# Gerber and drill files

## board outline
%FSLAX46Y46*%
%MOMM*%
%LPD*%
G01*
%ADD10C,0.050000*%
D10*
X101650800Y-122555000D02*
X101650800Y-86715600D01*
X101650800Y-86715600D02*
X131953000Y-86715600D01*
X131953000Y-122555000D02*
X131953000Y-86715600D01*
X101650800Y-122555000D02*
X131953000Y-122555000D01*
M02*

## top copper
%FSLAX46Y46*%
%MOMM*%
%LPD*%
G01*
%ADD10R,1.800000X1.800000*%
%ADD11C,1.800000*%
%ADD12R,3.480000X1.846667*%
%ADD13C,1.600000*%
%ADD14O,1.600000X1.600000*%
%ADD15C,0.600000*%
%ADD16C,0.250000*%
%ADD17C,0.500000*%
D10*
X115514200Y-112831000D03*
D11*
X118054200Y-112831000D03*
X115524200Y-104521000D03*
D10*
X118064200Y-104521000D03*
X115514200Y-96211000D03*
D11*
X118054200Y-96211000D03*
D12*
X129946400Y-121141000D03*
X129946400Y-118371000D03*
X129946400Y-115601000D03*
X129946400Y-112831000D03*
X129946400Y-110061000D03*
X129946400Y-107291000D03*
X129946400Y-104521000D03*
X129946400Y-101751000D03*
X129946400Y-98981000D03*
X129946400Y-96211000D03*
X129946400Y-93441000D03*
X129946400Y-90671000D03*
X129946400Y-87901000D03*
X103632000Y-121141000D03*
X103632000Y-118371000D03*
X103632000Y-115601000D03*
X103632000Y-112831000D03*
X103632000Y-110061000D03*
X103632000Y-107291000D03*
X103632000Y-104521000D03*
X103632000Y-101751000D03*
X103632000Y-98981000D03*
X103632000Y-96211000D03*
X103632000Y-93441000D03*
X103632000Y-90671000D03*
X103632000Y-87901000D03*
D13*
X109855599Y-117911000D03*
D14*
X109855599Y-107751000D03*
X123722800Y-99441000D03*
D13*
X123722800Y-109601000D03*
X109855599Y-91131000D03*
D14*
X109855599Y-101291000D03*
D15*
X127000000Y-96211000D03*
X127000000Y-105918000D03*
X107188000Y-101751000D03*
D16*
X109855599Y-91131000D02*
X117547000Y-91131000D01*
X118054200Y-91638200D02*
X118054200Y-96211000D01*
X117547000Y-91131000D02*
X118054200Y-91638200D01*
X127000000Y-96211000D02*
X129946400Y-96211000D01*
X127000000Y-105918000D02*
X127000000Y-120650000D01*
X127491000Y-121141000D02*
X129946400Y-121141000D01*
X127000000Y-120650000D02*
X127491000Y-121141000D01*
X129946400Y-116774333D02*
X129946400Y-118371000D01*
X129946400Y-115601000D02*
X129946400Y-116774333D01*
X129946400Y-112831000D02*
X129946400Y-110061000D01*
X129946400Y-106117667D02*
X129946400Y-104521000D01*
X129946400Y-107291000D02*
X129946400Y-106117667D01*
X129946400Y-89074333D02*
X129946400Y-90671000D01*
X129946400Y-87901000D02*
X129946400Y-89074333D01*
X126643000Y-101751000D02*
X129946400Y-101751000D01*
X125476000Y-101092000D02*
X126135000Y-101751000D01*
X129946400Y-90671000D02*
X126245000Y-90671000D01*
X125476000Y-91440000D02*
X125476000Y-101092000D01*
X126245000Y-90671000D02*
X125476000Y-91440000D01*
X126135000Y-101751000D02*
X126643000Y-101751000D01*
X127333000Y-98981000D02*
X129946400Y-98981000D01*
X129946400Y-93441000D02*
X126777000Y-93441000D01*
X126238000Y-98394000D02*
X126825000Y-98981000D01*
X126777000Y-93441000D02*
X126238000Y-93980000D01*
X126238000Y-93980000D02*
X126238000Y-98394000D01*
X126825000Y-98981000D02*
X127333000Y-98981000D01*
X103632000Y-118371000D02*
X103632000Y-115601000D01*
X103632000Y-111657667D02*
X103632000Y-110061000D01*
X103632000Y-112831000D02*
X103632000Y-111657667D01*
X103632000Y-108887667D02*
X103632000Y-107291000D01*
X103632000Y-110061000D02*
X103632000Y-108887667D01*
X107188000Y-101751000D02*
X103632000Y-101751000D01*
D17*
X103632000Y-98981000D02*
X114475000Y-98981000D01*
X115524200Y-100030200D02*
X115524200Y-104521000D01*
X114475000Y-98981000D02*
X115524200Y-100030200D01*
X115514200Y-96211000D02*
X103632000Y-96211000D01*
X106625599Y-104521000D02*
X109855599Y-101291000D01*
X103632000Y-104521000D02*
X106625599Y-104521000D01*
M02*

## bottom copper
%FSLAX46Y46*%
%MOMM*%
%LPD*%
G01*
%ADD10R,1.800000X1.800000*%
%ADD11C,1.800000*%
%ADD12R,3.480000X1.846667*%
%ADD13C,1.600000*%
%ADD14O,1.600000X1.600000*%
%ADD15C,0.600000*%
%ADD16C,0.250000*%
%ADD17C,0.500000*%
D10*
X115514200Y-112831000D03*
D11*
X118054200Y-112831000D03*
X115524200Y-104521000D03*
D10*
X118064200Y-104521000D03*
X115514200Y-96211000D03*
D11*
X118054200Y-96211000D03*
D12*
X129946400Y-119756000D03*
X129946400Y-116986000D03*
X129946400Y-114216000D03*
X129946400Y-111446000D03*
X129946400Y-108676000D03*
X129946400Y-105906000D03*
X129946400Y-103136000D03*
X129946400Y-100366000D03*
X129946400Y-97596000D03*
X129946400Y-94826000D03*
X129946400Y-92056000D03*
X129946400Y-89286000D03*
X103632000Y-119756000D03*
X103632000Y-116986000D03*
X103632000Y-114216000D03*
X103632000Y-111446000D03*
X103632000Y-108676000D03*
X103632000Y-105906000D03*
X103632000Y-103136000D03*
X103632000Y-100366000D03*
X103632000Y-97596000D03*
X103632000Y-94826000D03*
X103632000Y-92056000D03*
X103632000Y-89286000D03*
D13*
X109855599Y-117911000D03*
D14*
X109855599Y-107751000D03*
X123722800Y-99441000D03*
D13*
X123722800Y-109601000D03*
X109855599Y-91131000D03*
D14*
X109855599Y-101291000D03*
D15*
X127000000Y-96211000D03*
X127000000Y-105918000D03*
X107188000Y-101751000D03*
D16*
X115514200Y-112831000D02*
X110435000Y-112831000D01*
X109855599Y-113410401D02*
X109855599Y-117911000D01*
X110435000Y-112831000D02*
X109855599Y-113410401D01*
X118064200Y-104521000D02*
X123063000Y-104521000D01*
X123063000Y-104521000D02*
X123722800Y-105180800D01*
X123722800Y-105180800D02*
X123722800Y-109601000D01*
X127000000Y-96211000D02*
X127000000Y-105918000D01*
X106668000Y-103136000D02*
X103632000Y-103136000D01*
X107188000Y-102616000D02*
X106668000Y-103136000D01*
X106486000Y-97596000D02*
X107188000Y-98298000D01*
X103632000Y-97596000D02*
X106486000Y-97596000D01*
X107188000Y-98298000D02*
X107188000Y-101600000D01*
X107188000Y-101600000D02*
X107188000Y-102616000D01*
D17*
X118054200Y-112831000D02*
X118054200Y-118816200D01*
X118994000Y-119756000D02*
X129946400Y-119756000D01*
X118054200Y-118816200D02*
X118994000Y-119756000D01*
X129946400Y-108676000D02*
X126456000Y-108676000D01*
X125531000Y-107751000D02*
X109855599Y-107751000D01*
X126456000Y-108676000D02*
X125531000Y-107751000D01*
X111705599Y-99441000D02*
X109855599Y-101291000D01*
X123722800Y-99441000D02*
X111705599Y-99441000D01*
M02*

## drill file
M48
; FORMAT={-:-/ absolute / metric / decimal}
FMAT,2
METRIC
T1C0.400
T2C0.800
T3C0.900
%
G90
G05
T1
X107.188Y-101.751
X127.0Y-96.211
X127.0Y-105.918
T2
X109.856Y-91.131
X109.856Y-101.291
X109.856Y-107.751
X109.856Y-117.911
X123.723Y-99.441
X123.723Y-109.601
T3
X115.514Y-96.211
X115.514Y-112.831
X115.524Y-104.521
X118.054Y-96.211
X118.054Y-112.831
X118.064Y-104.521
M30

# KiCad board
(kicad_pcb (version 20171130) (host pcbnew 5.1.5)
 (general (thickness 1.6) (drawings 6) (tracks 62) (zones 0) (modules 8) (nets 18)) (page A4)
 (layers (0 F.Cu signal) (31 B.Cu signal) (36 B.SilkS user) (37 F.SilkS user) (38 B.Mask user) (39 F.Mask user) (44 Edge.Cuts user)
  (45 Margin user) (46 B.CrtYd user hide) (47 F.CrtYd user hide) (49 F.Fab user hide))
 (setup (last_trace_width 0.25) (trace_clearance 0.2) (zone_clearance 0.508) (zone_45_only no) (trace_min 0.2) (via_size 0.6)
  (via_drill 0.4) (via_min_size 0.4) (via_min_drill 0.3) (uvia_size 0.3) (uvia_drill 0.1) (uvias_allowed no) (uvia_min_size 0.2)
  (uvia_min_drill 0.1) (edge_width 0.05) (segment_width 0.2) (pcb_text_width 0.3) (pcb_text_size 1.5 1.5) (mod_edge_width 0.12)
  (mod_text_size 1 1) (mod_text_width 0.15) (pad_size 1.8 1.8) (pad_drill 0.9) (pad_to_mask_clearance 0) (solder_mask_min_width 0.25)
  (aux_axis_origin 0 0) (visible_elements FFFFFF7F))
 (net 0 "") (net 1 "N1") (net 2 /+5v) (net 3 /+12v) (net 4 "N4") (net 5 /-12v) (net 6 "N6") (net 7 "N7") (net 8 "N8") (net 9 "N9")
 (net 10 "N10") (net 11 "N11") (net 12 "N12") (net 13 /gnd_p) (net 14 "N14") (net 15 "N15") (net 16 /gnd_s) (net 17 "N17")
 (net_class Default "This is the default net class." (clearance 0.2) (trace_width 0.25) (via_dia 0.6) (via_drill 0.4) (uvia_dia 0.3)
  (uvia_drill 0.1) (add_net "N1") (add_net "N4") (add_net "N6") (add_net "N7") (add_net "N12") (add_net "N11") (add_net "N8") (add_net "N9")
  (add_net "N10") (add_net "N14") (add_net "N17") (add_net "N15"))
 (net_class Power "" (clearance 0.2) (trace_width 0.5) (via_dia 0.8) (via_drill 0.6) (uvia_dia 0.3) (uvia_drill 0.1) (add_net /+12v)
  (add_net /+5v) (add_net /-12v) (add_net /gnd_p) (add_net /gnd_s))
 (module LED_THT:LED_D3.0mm (layer F.Cu) (at 115.5142 112.831)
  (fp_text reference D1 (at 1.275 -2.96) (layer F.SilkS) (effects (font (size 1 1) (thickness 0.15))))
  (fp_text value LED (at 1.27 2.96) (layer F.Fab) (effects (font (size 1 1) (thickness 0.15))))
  (pad 1 thru_hole rect (at 0 0) (size 1.8 1.8) (drill 0.9) (layers *.Cu *.Mask) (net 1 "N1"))
  (pad 2 thru_hole circle (at 2.54 0) (size 1.8 1.8) (drill 0.9) (layers *.Cu *.Mask) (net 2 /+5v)))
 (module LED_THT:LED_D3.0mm (layer F.Cu) (at 118.0642 104.521 180)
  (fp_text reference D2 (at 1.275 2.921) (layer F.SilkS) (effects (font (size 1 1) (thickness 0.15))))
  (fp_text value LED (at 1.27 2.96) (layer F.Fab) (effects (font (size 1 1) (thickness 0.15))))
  (pad 2 thru_hole circle (at 2.54 0 180) (size 1.8 1.8) (drill 0.9) (layers *.Cu *.Mask) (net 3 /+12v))
  (pad 1 thru_hole rect (at 0 0 180) (size 1.8 1.8) (drill 0.9) (layers *.Cu *.Mask) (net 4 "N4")))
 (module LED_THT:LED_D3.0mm (layer F.Cu) (at 115.5142 96.211)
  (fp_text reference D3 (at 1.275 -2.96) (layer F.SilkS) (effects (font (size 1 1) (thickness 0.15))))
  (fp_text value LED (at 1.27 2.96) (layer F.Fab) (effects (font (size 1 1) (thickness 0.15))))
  (pad 1 thru_hole rect (at 0 0) (size 1.8 1.8) (drill 0.9) (layers *.Cu *.Mask) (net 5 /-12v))
  (pad 2 thru_hole circle (at 2.54 0) (size 1.8 1.8) (drill 0.9) (layers *.Cu *.Mask) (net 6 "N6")))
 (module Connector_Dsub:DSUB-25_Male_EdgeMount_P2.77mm (layer F.Cu) (at 129.9464 104.521 90)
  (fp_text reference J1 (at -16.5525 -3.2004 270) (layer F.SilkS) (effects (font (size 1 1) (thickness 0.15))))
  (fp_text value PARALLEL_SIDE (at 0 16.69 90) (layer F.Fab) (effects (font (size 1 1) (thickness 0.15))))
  (pad 1 smd rect (at -16.62 0 90) (size 1.846667 3.48) (layers F.Cu F.Paste F.Mask) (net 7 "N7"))
  (pad 2 smd rect (at -13.85 0 90) (size 1.846667 3.48) (layers F.Cu F.Paste F.Mask) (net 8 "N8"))
  (pad 3 smd rect (at -11.08 0 90) (size 1.846667 3.48) (layers F.Cu F.Paste F.Mask) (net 8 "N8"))
  (pad 4 smd rect (at -8.31 0 90) (size 1.846667 3.48) (layers F.Cu F.Paste F.Mask) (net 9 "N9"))
  (pad 5 smd rect (at -5.54 0 90) (size 1.846667 3.48) (layers F.Cu F.Paste F.Mask) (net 9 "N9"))
  (pad 6 smd rect (at -2.77 0 90) (size 1.846667 3.48) (layers F.Cu F.Paste F.Mask) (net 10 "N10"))
  (pad 7 smd rect (at 0 0 90) (size 1.846667 3.48) (layers F.Cu F.Paste F.Mask) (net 10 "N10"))
  (pad 8 smd rect (at 2.77 0 90) (size 1.846667 3.48) (layers F.Cu F.Paste F.Mask) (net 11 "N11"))
  (pad 9 smd rect (at 5.54 0 90) (size 1.846667 3.48) (layers F.Cu F.Paste F.Mask) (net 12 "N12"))
  (pad 10 smd rect (at 8.31 0 90) (size 1.846667 3.48) (layers F.Cu F.Paste F.Mask) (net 7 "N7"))
  (pad 11 smd rect (at 11.08 0 90) (size 1.846667 3.48) (layers F.Cu F.Paste F.Mask) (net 12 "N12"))
  (pad 12 smd rect (at 13.85 0 90) (size 1.846667 3.48) (layers F.Cu F.Paste F.Mask) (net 11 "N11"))
  (pad 13 smd rect (at 16.62 0 90) (size 1.846667 3.48) (layers F.Cu F.Paste F.Mask) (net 11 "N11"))
  (pad 14 smd rect (at -15.235 0 90) (size 1.846667 3.48) (layers B.Cu B.Paste B.Mask) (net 2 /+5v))
  (pad 15 smd rect (at -12.465 0 90) (size 1.846667 3.48) (layers B.Cu B.Paste B.Mask))
  (pad 16 smd rect (at -9.695 0 90) (size 1.846667 3.48) (layers B.Cu B.Paste B.Mask))
  (pad 17 smd rect (at -6.925 0 90) (size 1.846667 3.48) (layers B.Cu B.Paste B.Mask))
  (pad 18 smd rect (at -4.155 0 90) (size 1.846667 3.48) (layers B.Cu B.Paste B.Mask) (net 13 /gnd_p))
  (pad 19 smd rect (at -1.385 0 90) (size 1.846667 3.48) (layers B.Cu B.Paste B.Mask))
  (pad 20 smd rect (at 1.385 0 90) (size 1.846667 3.48) (layers B.Cu B.Paste B.Mask))
  (pad 21 smd rect (at 4.155 0 90) (size 1.846667 3.48) (layers B.Cu B.Paste B.Mask))
  (pad 22 smd rect (at 6.925 0 90) (size 1.846667 3.48) (layers B.Cu B.Paste B.Mask))
  (pad 23 smd rect (at 9.695 0 90) (size 1.846667 3.48) (layers B.Cu B.Paste B.Mask))
  (pad 24 smd rect (at 12.465 0 90) (size 1.846667 3.48) (layers B.Cu B.Paste B.Mask))
  (pad 25 smd rect (at 15.235 0 90) (size 1.846667 3.48) (layers B.Cu B.Paste B.Mask)))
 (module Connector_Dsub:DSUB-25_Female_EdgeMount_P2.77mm (layer F.Cu) (at 103.632 104.521 270)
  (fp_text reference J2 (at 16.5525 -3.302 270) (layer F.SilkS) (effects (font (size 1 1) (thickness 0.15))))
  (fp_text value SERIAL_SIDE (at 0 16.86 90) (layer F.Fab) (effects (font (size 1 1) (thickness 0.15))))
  (pad 1 smd rect (at 16.62 0 270) (size 1.846667 3.48) (layers F.Cu F.Paste F.Mask))
  (pad 2 smd rect (at 13.85 0 270) (size 1.846667 3.48) (layers F.Cu F.Paste F.Mask) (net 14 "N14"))
  (pad 3 smd rect (at 11.08 0 270) (size 1.846667 3.48) (layers F.Cu F.Paste F.Mask) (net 14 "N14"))
  (pad 4 smd rect (at 8.31 0 270) (size 1.846667 3.48) (layers F.Cu F.Paste F.Mask) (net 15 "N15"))
  (pad 5 smd rect (at 5.54 0 270) (size 1.846667 3.48) (layers F.Cu F.Paste F.Mask) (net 15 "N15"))
  (pad 6 smd rect (at 2.77 0 270) (size 1.846667 3.48) (layers F.Cu F.Paste F.Mask) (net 15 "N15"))
  (pad 7 smd rect (at 0 0 270) (size 1.846667 3.48) (layers F.Cu F.Paste F.Mask) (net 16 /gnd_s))
  (pad 8 smd rect (at -2.77 0 270) (size 1.846667 3.48) (layers F.Cu F.Paste F.Mask) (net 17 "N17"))
  (pad 9 smd rect (at -5.54 0 270) (size 1.846667 3.48) (layers F.Cu F.Paste F.Mask) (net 3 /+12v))
  (pad 10 smd rect (at -8.31 0 270) (size 1.846667 3.48) (layers F.Cu F.Paste F.Mask) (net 5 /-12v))
  (pad 11 smd rect (at -11.08 0 270) (size 1.846667 3.48) (layers F.Cu F.Paste F.Mask))
  (pad 12 smd rect (at -13.85 0 270) (size 1.846667 3.48) (layers F.Cu F.Paste F.Mask))
  (pad 13 smd rect (at -16.62 0 270) (size 1.846667 3.48) (layers F.Cu F.Paste F.Mask))
  (pad 14 smd rect (at 15.235 0 270) (size 1.846667 3.48) (layers B.Cu B.Paste B.Mask))
  (pad 15 smd rect (at 12.465 0 270) (size 1.846667 3.48) (layers B.Cu B.Paste B.Mask))
  (pad 16 smd rect (at 9.695 0 270) (size 1.846667 3.48) (layers B.Cu B.Paste B.Mask))
  (pad 17 smd rect (at 6.925 0 270) (size 1.846667 3.48) (layers B.Cu B.Paste B.Mask))
  (pad 18 smd rect (at 4.155 0 270) (size 1.846667 3.48) (layers B.Cu B.Paste B.Mask))
  (pad 19 smd rect (at 1.385 0 270) (size 1.846667 3.48) (layers B.Cu B.Paste B.Mask))
  (pad 20 smd rect (at -1.385 0 270) (size 1.846667 3.48) (layers B.Cu B.Paste B.Mask) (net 17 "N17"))
  (pad 21 smd rect (at -4.155 0 270) (size 1.846667 3.48) (layers B.Cu B.Paste B.Mask))
  (pad 22 smd rect (at -6.925 0 270) (size 1.846667 3.48) (layers B.Cu B.Paste B.Mask) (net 17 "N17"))
  (pad 23 smd rect (at -9.695 0 270) (size 1.846667 3.48) (layers B.Cu B.Paste B.Mask))
  (pad 24 smd rect (at -12.465 0 270) (size 1.846667 3.48) (layers B.Cu B.Paste B.Mask))
  (pad 25 smd rect (at -15.235 0 270) (size 1.846667 3.48) (layers B.Cu B.Paste B.Mask)))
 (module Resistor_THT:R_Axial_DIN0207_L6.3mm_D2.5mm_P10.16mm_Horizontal (layer F.Cu) (at 109.855599 117.911 90)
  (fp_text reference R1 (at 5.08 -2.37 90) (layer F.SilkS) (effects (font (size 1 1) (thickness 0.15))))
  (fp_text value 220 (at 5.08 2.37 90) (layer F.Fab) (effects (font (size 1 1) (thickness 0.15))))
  (pad 1 thru_hole circle (at 0 0 90) (size 1.6 1.6) (drill 0.8) (layers *.Cu *.Mask) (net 1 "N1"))
  (pad 2 thru_hole oval (at 10.16 0 90) (size 1.6 1.6) (drill 0.8) (layers *.Cu *.Mask) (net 13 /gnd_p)))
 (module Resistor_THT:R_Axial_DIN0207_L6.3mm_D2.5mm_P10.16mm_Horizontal (layer F.Cu) (at 123.7228 109.601 90)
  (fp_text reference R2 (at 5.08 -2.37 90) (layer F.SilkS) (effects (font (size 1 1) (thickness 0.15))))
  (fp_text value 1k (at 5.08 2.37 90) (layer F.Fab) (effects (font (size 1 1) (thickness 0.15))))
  (pad 2 thru_hole oval (at 10.16 0 90) (size 1.6 1.6) (drill 0.8) (layers *.Cu *.Mask) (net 16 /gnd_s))
  (pad 1 thru_hole circle (at 0 0 90) (size 1.6 1.6) (drill 0.8) (layers *.Cu *.Mask) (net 4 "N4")))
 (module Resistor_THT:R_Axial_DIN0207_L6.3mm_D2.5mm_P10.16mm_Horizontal (layer F.Cu) (at 109.855599 91.131 270)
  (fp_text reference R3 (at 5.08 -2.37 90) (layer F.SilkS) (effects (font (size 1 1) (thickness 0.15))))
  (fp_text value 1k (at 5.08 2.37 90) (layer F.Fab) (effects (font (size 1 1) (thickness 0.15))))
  (pad 1 thru_hole circle (at 0 0 270) (size 1.6 1.6) (drill 0.8) (layers *.Cu *.Mask) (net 6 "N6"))
  (pad 2 thru_hole oval (at 10.16 0 270) (size 1.6 1.6) (drill 0.8) (layers *.Cu *.Mask) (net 16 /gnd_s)))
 (gr_line (start 101.6508 122.555) (end 101.6508 86.7156) (layer Edge.Cuts) (width 0.05))
 (gr_line (start 101.6508 86.7156) (end 131.953 86.7156) (layer Edge.Cuts) (width 0.05))
 (gr_line (start 131.953 122.555) (end 131.953 86.7156) (layer Edge.Cuts) (width 0.05))
 (gr_line (start 101.6508 122.555) (end 131.953 122.555) (layer Edge.Cuts) (width 0.05))
 (segment (start 115.5142 112.831) (end 110.435 112.831) (width 0.25) (layer B.Cu) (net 1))
 (segment (start 109.855599 113.410401) (end 109.855599 117.911) (width 0.25) (layer B.Cu) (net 1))
 (segment (start 110.435 112.831) (end 109.855599 113.410401) (width 0.25) (layer B.Cu) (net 1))
 (segment (start 118.0642 104.521) (end 123.063 104.521) (width 0.25) (layer B.Cu) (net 4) (status 1000000))
 (segment (start 123.063 104.521) (end 123.7228 105.1808) (width 0.25) (layer B.Cu) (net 4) (status 1000000))
 (segment (start 123.7228 105.1808) (end 123.7228 109.601) (width 0.25) (layer B.Cu) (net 4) (status 1000000))
 (segment (start 109.855599 91.131) (end 117.547 91.131) (width 0.25) (layer F.Cu) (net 6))
 (segment (start 118.0542 91.6382) (end 118.0542 96.211) (width 0.25) (layer F.Cu) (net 6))
 (segment (start 117.547 91.131) (end 118.0542 91.6382) (width 0.25) (layer F.Cu) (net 6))
 (via (at 127 96.211) (size 0.6) (drill 0.4) (layers F.Cu B.Cu) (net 7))
 (segment (start 127 96.211) (end 129.9464 96.211) (width 0.25) (layer F.Cu) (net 7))
 (via (at 127 105.918) (size 0.6) (drill 0.4) (layers F.Cu B.Cu) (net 7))
 (segment (start 127 96.211) (end 127 105.918) (width 0.25) (layer B.Cu) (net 7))
 (segment (start 127 105.918) (end 127 120.65) (width 0.25) (layer F.Cu) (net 7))
 (segment (start 127.491 121.141) (end 129.9464 121.141) (width 0.25) (layer F.Cu) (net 7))
 (segment (start 127 120.65) (end 127.491 121.141) (width 0.25) (layer F.Cu) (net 7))
 (segment (start 129.9464 116.774333) (end 129.9464 118.371) (width 0.25) (layer F.Cu) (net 8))
 (segment (start 129.9464 115.601) (end 129.9464 116.774333) (width 0.25) (layer F.Cu) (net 8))
 (segment (start 129.9464 112.831) (end 129.9464 110.061) (width 0.25) (layer F.Cu) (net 9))
 (segment (start 129.9464 106.117667) (end 129.9464 104.521) (width 0.25) (layer F.Cu) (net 10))
 (segment (start 129.9464 107.291) (end 129.9464 106.117667) (width 0.25) (layer F.Cu) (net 10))
 (segment (start 129.9464 89.074333) (end 129.9464 90.671) (width 0.25) (layer F.Cu) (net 11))
 (segment (start 129.9464 87.901) (end 129.9464 89.074333) (width 0.25) (layer F.Cu) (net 11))
 (segment (start 126.643 101.751) (end 129.9464 101.751) (width 0.25) (layer F.Cu) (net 11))
 (segment (start 125.476 101.092) (end 126.135 101.751) (width 0.25) (layer F.Cu) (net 11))
 (segment (start 129.9464 90.671) (end 126.245 90.671) (width 0.25) (layer F.Cu) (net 11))
 (segment (start 125.476 91.44) (end 125.476 101.092) (width 0.25) (layer F.Cu) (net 11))
 (segment (start 126.245 90.671) (end 125.476 91.44) (width 0.25) (layer F.Cu) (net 11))
 (segment (start 126.135 101.751) (end 126.643 101.751) (width 0.25) (layer F.Cu) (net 11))
 (segment (start 127.333 98.981) (end 129.9464 98.981) (width 0.25) (layer F.Cu) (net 12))
 (segment (start 129.9464 93.441) (end 126.777 93.441) (width 0.25) (layer F.Cu) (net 12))
 (segment (start 126.238 98.394) (end 126.825 98.981) (width 0.25) (layer F.Cu) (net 12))
 (segment (start 126.777 93.441) (end 126.238 93.98) (width 0.25) (layer F.Cu) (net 12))
 (segment (start 126.238 93.98) (end 126.238 98.394) (width 0.25) (layer F.Cu) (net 12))
 (segment (start 126.825 98.981) (end 127.333 98.981) (width 0.25) (layer F.Cu) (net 12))
 (segment (start 103.632 118.371) (end 103.632 115.601) (width 0.25) (layer F.Cu) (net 14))
 (segment (start 103.632 111.657667) (end 103.632 110.061) (width 0.25) (layer F.Cu) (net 15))
 (segment (start 103.632 112.831) (end 103.632 111.657667) (width 0.25) (layer F.Cu) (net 15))
 (segment (start 103.632 108.887667) (end 103.632 107.291) (width 0.25) (layer F.Cu) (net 15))
 (segment (start 103.632 110.061) (end 103.632 108.887667) (width 0.25) (layer F.Cu) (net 15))
 (segment (start 106.668 103.136) (end 103.632 103.136) (width 0.25) (layer B.Cu) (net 17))
 (segment (start 107.188 102.616) (end 106.668 103.136) (width 0.25) (layer B.Cu) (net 17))
 (segment (start 106.486 97.596) (end 107.188 98.298) (width 0.25) (layer B.Cu) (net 17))
 (segment (start 103.632 97.596) (end 106.486 97.596) (width 0.25) (layer B.Cu) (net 17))
 (via (at 107.188 101.751) (size 0.6) (drill 0.4) (layers F.Cu B.Cu) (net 17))
 (segment (start 107.188 98.298) (end 107.188 101.6) (width 0.25) (layer B.Cu) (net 17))
 (segment (start 107.188 101.6) (end 107.188 102.616) (width 0.25) (layer B.Cu) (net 17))
 (segment (start 107.188 101.751) (end 103.632 101.751) (width 0.25) (layer F.Cu) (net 17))
 (segment (start 118.0542 112.831) (end 118.0542 118.8162) (width 0.5) (layer B.Cu) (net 2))
 (segment (start 118.994 119.756) (end 129.9464 119.756) (width 0.5) (layer B.Cu) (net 2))
 (segment (start 118.0542 118.8162) (end 118.994 119.756) (width 0.5) (layer B.Cu) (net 2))
 (segment (start 103.632 98.981) (end 114.475 98.981) (width 0.5) (layer F.Cu) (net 3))
 (segment (start 115.5242 100.0302) (end 115.5242 104.521) (width 0.5) (layer F.Cu) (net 3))
 (segment (start 114.475 98.981) (end 115.5242 100.0302) (width 0.5) (layer F.Cu) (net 3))
 (segment (start 115.5142 96.211) (end 103.632 96.211) (width 0.5) (layer F.Cu) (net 5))
 (segment (start 129.9464 108.676) (end 126.456 108.676) (width 0.5) (layer B.Cu) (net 13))
 (segment (start 125.531 107.751) (end 109.855599 107.751) (width 0.5) (layer B.Cu) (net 13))
 (segment (start 126.456 108.676) (end 125.531 107.751) (width 0.5) (layer B.Cu) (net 13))
 (segment (start 106.625599 104.521) (end 109.855599 101.291) (width 0.5) (layer F.Cu) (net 16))
 (segment (start 103.632 104.521) (end 106.625599 104.521) (width 0.5) (layer F.Cu) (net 16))
 (segment (start 111.705599 99.441) (end 109.855599 101.291) (width 0.5) (layer B.Cu) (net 16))
 (segment (start 123.7228 99.441) (end 111.705599 99.441) (width 0.5) (layer B.Cu) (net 16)))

